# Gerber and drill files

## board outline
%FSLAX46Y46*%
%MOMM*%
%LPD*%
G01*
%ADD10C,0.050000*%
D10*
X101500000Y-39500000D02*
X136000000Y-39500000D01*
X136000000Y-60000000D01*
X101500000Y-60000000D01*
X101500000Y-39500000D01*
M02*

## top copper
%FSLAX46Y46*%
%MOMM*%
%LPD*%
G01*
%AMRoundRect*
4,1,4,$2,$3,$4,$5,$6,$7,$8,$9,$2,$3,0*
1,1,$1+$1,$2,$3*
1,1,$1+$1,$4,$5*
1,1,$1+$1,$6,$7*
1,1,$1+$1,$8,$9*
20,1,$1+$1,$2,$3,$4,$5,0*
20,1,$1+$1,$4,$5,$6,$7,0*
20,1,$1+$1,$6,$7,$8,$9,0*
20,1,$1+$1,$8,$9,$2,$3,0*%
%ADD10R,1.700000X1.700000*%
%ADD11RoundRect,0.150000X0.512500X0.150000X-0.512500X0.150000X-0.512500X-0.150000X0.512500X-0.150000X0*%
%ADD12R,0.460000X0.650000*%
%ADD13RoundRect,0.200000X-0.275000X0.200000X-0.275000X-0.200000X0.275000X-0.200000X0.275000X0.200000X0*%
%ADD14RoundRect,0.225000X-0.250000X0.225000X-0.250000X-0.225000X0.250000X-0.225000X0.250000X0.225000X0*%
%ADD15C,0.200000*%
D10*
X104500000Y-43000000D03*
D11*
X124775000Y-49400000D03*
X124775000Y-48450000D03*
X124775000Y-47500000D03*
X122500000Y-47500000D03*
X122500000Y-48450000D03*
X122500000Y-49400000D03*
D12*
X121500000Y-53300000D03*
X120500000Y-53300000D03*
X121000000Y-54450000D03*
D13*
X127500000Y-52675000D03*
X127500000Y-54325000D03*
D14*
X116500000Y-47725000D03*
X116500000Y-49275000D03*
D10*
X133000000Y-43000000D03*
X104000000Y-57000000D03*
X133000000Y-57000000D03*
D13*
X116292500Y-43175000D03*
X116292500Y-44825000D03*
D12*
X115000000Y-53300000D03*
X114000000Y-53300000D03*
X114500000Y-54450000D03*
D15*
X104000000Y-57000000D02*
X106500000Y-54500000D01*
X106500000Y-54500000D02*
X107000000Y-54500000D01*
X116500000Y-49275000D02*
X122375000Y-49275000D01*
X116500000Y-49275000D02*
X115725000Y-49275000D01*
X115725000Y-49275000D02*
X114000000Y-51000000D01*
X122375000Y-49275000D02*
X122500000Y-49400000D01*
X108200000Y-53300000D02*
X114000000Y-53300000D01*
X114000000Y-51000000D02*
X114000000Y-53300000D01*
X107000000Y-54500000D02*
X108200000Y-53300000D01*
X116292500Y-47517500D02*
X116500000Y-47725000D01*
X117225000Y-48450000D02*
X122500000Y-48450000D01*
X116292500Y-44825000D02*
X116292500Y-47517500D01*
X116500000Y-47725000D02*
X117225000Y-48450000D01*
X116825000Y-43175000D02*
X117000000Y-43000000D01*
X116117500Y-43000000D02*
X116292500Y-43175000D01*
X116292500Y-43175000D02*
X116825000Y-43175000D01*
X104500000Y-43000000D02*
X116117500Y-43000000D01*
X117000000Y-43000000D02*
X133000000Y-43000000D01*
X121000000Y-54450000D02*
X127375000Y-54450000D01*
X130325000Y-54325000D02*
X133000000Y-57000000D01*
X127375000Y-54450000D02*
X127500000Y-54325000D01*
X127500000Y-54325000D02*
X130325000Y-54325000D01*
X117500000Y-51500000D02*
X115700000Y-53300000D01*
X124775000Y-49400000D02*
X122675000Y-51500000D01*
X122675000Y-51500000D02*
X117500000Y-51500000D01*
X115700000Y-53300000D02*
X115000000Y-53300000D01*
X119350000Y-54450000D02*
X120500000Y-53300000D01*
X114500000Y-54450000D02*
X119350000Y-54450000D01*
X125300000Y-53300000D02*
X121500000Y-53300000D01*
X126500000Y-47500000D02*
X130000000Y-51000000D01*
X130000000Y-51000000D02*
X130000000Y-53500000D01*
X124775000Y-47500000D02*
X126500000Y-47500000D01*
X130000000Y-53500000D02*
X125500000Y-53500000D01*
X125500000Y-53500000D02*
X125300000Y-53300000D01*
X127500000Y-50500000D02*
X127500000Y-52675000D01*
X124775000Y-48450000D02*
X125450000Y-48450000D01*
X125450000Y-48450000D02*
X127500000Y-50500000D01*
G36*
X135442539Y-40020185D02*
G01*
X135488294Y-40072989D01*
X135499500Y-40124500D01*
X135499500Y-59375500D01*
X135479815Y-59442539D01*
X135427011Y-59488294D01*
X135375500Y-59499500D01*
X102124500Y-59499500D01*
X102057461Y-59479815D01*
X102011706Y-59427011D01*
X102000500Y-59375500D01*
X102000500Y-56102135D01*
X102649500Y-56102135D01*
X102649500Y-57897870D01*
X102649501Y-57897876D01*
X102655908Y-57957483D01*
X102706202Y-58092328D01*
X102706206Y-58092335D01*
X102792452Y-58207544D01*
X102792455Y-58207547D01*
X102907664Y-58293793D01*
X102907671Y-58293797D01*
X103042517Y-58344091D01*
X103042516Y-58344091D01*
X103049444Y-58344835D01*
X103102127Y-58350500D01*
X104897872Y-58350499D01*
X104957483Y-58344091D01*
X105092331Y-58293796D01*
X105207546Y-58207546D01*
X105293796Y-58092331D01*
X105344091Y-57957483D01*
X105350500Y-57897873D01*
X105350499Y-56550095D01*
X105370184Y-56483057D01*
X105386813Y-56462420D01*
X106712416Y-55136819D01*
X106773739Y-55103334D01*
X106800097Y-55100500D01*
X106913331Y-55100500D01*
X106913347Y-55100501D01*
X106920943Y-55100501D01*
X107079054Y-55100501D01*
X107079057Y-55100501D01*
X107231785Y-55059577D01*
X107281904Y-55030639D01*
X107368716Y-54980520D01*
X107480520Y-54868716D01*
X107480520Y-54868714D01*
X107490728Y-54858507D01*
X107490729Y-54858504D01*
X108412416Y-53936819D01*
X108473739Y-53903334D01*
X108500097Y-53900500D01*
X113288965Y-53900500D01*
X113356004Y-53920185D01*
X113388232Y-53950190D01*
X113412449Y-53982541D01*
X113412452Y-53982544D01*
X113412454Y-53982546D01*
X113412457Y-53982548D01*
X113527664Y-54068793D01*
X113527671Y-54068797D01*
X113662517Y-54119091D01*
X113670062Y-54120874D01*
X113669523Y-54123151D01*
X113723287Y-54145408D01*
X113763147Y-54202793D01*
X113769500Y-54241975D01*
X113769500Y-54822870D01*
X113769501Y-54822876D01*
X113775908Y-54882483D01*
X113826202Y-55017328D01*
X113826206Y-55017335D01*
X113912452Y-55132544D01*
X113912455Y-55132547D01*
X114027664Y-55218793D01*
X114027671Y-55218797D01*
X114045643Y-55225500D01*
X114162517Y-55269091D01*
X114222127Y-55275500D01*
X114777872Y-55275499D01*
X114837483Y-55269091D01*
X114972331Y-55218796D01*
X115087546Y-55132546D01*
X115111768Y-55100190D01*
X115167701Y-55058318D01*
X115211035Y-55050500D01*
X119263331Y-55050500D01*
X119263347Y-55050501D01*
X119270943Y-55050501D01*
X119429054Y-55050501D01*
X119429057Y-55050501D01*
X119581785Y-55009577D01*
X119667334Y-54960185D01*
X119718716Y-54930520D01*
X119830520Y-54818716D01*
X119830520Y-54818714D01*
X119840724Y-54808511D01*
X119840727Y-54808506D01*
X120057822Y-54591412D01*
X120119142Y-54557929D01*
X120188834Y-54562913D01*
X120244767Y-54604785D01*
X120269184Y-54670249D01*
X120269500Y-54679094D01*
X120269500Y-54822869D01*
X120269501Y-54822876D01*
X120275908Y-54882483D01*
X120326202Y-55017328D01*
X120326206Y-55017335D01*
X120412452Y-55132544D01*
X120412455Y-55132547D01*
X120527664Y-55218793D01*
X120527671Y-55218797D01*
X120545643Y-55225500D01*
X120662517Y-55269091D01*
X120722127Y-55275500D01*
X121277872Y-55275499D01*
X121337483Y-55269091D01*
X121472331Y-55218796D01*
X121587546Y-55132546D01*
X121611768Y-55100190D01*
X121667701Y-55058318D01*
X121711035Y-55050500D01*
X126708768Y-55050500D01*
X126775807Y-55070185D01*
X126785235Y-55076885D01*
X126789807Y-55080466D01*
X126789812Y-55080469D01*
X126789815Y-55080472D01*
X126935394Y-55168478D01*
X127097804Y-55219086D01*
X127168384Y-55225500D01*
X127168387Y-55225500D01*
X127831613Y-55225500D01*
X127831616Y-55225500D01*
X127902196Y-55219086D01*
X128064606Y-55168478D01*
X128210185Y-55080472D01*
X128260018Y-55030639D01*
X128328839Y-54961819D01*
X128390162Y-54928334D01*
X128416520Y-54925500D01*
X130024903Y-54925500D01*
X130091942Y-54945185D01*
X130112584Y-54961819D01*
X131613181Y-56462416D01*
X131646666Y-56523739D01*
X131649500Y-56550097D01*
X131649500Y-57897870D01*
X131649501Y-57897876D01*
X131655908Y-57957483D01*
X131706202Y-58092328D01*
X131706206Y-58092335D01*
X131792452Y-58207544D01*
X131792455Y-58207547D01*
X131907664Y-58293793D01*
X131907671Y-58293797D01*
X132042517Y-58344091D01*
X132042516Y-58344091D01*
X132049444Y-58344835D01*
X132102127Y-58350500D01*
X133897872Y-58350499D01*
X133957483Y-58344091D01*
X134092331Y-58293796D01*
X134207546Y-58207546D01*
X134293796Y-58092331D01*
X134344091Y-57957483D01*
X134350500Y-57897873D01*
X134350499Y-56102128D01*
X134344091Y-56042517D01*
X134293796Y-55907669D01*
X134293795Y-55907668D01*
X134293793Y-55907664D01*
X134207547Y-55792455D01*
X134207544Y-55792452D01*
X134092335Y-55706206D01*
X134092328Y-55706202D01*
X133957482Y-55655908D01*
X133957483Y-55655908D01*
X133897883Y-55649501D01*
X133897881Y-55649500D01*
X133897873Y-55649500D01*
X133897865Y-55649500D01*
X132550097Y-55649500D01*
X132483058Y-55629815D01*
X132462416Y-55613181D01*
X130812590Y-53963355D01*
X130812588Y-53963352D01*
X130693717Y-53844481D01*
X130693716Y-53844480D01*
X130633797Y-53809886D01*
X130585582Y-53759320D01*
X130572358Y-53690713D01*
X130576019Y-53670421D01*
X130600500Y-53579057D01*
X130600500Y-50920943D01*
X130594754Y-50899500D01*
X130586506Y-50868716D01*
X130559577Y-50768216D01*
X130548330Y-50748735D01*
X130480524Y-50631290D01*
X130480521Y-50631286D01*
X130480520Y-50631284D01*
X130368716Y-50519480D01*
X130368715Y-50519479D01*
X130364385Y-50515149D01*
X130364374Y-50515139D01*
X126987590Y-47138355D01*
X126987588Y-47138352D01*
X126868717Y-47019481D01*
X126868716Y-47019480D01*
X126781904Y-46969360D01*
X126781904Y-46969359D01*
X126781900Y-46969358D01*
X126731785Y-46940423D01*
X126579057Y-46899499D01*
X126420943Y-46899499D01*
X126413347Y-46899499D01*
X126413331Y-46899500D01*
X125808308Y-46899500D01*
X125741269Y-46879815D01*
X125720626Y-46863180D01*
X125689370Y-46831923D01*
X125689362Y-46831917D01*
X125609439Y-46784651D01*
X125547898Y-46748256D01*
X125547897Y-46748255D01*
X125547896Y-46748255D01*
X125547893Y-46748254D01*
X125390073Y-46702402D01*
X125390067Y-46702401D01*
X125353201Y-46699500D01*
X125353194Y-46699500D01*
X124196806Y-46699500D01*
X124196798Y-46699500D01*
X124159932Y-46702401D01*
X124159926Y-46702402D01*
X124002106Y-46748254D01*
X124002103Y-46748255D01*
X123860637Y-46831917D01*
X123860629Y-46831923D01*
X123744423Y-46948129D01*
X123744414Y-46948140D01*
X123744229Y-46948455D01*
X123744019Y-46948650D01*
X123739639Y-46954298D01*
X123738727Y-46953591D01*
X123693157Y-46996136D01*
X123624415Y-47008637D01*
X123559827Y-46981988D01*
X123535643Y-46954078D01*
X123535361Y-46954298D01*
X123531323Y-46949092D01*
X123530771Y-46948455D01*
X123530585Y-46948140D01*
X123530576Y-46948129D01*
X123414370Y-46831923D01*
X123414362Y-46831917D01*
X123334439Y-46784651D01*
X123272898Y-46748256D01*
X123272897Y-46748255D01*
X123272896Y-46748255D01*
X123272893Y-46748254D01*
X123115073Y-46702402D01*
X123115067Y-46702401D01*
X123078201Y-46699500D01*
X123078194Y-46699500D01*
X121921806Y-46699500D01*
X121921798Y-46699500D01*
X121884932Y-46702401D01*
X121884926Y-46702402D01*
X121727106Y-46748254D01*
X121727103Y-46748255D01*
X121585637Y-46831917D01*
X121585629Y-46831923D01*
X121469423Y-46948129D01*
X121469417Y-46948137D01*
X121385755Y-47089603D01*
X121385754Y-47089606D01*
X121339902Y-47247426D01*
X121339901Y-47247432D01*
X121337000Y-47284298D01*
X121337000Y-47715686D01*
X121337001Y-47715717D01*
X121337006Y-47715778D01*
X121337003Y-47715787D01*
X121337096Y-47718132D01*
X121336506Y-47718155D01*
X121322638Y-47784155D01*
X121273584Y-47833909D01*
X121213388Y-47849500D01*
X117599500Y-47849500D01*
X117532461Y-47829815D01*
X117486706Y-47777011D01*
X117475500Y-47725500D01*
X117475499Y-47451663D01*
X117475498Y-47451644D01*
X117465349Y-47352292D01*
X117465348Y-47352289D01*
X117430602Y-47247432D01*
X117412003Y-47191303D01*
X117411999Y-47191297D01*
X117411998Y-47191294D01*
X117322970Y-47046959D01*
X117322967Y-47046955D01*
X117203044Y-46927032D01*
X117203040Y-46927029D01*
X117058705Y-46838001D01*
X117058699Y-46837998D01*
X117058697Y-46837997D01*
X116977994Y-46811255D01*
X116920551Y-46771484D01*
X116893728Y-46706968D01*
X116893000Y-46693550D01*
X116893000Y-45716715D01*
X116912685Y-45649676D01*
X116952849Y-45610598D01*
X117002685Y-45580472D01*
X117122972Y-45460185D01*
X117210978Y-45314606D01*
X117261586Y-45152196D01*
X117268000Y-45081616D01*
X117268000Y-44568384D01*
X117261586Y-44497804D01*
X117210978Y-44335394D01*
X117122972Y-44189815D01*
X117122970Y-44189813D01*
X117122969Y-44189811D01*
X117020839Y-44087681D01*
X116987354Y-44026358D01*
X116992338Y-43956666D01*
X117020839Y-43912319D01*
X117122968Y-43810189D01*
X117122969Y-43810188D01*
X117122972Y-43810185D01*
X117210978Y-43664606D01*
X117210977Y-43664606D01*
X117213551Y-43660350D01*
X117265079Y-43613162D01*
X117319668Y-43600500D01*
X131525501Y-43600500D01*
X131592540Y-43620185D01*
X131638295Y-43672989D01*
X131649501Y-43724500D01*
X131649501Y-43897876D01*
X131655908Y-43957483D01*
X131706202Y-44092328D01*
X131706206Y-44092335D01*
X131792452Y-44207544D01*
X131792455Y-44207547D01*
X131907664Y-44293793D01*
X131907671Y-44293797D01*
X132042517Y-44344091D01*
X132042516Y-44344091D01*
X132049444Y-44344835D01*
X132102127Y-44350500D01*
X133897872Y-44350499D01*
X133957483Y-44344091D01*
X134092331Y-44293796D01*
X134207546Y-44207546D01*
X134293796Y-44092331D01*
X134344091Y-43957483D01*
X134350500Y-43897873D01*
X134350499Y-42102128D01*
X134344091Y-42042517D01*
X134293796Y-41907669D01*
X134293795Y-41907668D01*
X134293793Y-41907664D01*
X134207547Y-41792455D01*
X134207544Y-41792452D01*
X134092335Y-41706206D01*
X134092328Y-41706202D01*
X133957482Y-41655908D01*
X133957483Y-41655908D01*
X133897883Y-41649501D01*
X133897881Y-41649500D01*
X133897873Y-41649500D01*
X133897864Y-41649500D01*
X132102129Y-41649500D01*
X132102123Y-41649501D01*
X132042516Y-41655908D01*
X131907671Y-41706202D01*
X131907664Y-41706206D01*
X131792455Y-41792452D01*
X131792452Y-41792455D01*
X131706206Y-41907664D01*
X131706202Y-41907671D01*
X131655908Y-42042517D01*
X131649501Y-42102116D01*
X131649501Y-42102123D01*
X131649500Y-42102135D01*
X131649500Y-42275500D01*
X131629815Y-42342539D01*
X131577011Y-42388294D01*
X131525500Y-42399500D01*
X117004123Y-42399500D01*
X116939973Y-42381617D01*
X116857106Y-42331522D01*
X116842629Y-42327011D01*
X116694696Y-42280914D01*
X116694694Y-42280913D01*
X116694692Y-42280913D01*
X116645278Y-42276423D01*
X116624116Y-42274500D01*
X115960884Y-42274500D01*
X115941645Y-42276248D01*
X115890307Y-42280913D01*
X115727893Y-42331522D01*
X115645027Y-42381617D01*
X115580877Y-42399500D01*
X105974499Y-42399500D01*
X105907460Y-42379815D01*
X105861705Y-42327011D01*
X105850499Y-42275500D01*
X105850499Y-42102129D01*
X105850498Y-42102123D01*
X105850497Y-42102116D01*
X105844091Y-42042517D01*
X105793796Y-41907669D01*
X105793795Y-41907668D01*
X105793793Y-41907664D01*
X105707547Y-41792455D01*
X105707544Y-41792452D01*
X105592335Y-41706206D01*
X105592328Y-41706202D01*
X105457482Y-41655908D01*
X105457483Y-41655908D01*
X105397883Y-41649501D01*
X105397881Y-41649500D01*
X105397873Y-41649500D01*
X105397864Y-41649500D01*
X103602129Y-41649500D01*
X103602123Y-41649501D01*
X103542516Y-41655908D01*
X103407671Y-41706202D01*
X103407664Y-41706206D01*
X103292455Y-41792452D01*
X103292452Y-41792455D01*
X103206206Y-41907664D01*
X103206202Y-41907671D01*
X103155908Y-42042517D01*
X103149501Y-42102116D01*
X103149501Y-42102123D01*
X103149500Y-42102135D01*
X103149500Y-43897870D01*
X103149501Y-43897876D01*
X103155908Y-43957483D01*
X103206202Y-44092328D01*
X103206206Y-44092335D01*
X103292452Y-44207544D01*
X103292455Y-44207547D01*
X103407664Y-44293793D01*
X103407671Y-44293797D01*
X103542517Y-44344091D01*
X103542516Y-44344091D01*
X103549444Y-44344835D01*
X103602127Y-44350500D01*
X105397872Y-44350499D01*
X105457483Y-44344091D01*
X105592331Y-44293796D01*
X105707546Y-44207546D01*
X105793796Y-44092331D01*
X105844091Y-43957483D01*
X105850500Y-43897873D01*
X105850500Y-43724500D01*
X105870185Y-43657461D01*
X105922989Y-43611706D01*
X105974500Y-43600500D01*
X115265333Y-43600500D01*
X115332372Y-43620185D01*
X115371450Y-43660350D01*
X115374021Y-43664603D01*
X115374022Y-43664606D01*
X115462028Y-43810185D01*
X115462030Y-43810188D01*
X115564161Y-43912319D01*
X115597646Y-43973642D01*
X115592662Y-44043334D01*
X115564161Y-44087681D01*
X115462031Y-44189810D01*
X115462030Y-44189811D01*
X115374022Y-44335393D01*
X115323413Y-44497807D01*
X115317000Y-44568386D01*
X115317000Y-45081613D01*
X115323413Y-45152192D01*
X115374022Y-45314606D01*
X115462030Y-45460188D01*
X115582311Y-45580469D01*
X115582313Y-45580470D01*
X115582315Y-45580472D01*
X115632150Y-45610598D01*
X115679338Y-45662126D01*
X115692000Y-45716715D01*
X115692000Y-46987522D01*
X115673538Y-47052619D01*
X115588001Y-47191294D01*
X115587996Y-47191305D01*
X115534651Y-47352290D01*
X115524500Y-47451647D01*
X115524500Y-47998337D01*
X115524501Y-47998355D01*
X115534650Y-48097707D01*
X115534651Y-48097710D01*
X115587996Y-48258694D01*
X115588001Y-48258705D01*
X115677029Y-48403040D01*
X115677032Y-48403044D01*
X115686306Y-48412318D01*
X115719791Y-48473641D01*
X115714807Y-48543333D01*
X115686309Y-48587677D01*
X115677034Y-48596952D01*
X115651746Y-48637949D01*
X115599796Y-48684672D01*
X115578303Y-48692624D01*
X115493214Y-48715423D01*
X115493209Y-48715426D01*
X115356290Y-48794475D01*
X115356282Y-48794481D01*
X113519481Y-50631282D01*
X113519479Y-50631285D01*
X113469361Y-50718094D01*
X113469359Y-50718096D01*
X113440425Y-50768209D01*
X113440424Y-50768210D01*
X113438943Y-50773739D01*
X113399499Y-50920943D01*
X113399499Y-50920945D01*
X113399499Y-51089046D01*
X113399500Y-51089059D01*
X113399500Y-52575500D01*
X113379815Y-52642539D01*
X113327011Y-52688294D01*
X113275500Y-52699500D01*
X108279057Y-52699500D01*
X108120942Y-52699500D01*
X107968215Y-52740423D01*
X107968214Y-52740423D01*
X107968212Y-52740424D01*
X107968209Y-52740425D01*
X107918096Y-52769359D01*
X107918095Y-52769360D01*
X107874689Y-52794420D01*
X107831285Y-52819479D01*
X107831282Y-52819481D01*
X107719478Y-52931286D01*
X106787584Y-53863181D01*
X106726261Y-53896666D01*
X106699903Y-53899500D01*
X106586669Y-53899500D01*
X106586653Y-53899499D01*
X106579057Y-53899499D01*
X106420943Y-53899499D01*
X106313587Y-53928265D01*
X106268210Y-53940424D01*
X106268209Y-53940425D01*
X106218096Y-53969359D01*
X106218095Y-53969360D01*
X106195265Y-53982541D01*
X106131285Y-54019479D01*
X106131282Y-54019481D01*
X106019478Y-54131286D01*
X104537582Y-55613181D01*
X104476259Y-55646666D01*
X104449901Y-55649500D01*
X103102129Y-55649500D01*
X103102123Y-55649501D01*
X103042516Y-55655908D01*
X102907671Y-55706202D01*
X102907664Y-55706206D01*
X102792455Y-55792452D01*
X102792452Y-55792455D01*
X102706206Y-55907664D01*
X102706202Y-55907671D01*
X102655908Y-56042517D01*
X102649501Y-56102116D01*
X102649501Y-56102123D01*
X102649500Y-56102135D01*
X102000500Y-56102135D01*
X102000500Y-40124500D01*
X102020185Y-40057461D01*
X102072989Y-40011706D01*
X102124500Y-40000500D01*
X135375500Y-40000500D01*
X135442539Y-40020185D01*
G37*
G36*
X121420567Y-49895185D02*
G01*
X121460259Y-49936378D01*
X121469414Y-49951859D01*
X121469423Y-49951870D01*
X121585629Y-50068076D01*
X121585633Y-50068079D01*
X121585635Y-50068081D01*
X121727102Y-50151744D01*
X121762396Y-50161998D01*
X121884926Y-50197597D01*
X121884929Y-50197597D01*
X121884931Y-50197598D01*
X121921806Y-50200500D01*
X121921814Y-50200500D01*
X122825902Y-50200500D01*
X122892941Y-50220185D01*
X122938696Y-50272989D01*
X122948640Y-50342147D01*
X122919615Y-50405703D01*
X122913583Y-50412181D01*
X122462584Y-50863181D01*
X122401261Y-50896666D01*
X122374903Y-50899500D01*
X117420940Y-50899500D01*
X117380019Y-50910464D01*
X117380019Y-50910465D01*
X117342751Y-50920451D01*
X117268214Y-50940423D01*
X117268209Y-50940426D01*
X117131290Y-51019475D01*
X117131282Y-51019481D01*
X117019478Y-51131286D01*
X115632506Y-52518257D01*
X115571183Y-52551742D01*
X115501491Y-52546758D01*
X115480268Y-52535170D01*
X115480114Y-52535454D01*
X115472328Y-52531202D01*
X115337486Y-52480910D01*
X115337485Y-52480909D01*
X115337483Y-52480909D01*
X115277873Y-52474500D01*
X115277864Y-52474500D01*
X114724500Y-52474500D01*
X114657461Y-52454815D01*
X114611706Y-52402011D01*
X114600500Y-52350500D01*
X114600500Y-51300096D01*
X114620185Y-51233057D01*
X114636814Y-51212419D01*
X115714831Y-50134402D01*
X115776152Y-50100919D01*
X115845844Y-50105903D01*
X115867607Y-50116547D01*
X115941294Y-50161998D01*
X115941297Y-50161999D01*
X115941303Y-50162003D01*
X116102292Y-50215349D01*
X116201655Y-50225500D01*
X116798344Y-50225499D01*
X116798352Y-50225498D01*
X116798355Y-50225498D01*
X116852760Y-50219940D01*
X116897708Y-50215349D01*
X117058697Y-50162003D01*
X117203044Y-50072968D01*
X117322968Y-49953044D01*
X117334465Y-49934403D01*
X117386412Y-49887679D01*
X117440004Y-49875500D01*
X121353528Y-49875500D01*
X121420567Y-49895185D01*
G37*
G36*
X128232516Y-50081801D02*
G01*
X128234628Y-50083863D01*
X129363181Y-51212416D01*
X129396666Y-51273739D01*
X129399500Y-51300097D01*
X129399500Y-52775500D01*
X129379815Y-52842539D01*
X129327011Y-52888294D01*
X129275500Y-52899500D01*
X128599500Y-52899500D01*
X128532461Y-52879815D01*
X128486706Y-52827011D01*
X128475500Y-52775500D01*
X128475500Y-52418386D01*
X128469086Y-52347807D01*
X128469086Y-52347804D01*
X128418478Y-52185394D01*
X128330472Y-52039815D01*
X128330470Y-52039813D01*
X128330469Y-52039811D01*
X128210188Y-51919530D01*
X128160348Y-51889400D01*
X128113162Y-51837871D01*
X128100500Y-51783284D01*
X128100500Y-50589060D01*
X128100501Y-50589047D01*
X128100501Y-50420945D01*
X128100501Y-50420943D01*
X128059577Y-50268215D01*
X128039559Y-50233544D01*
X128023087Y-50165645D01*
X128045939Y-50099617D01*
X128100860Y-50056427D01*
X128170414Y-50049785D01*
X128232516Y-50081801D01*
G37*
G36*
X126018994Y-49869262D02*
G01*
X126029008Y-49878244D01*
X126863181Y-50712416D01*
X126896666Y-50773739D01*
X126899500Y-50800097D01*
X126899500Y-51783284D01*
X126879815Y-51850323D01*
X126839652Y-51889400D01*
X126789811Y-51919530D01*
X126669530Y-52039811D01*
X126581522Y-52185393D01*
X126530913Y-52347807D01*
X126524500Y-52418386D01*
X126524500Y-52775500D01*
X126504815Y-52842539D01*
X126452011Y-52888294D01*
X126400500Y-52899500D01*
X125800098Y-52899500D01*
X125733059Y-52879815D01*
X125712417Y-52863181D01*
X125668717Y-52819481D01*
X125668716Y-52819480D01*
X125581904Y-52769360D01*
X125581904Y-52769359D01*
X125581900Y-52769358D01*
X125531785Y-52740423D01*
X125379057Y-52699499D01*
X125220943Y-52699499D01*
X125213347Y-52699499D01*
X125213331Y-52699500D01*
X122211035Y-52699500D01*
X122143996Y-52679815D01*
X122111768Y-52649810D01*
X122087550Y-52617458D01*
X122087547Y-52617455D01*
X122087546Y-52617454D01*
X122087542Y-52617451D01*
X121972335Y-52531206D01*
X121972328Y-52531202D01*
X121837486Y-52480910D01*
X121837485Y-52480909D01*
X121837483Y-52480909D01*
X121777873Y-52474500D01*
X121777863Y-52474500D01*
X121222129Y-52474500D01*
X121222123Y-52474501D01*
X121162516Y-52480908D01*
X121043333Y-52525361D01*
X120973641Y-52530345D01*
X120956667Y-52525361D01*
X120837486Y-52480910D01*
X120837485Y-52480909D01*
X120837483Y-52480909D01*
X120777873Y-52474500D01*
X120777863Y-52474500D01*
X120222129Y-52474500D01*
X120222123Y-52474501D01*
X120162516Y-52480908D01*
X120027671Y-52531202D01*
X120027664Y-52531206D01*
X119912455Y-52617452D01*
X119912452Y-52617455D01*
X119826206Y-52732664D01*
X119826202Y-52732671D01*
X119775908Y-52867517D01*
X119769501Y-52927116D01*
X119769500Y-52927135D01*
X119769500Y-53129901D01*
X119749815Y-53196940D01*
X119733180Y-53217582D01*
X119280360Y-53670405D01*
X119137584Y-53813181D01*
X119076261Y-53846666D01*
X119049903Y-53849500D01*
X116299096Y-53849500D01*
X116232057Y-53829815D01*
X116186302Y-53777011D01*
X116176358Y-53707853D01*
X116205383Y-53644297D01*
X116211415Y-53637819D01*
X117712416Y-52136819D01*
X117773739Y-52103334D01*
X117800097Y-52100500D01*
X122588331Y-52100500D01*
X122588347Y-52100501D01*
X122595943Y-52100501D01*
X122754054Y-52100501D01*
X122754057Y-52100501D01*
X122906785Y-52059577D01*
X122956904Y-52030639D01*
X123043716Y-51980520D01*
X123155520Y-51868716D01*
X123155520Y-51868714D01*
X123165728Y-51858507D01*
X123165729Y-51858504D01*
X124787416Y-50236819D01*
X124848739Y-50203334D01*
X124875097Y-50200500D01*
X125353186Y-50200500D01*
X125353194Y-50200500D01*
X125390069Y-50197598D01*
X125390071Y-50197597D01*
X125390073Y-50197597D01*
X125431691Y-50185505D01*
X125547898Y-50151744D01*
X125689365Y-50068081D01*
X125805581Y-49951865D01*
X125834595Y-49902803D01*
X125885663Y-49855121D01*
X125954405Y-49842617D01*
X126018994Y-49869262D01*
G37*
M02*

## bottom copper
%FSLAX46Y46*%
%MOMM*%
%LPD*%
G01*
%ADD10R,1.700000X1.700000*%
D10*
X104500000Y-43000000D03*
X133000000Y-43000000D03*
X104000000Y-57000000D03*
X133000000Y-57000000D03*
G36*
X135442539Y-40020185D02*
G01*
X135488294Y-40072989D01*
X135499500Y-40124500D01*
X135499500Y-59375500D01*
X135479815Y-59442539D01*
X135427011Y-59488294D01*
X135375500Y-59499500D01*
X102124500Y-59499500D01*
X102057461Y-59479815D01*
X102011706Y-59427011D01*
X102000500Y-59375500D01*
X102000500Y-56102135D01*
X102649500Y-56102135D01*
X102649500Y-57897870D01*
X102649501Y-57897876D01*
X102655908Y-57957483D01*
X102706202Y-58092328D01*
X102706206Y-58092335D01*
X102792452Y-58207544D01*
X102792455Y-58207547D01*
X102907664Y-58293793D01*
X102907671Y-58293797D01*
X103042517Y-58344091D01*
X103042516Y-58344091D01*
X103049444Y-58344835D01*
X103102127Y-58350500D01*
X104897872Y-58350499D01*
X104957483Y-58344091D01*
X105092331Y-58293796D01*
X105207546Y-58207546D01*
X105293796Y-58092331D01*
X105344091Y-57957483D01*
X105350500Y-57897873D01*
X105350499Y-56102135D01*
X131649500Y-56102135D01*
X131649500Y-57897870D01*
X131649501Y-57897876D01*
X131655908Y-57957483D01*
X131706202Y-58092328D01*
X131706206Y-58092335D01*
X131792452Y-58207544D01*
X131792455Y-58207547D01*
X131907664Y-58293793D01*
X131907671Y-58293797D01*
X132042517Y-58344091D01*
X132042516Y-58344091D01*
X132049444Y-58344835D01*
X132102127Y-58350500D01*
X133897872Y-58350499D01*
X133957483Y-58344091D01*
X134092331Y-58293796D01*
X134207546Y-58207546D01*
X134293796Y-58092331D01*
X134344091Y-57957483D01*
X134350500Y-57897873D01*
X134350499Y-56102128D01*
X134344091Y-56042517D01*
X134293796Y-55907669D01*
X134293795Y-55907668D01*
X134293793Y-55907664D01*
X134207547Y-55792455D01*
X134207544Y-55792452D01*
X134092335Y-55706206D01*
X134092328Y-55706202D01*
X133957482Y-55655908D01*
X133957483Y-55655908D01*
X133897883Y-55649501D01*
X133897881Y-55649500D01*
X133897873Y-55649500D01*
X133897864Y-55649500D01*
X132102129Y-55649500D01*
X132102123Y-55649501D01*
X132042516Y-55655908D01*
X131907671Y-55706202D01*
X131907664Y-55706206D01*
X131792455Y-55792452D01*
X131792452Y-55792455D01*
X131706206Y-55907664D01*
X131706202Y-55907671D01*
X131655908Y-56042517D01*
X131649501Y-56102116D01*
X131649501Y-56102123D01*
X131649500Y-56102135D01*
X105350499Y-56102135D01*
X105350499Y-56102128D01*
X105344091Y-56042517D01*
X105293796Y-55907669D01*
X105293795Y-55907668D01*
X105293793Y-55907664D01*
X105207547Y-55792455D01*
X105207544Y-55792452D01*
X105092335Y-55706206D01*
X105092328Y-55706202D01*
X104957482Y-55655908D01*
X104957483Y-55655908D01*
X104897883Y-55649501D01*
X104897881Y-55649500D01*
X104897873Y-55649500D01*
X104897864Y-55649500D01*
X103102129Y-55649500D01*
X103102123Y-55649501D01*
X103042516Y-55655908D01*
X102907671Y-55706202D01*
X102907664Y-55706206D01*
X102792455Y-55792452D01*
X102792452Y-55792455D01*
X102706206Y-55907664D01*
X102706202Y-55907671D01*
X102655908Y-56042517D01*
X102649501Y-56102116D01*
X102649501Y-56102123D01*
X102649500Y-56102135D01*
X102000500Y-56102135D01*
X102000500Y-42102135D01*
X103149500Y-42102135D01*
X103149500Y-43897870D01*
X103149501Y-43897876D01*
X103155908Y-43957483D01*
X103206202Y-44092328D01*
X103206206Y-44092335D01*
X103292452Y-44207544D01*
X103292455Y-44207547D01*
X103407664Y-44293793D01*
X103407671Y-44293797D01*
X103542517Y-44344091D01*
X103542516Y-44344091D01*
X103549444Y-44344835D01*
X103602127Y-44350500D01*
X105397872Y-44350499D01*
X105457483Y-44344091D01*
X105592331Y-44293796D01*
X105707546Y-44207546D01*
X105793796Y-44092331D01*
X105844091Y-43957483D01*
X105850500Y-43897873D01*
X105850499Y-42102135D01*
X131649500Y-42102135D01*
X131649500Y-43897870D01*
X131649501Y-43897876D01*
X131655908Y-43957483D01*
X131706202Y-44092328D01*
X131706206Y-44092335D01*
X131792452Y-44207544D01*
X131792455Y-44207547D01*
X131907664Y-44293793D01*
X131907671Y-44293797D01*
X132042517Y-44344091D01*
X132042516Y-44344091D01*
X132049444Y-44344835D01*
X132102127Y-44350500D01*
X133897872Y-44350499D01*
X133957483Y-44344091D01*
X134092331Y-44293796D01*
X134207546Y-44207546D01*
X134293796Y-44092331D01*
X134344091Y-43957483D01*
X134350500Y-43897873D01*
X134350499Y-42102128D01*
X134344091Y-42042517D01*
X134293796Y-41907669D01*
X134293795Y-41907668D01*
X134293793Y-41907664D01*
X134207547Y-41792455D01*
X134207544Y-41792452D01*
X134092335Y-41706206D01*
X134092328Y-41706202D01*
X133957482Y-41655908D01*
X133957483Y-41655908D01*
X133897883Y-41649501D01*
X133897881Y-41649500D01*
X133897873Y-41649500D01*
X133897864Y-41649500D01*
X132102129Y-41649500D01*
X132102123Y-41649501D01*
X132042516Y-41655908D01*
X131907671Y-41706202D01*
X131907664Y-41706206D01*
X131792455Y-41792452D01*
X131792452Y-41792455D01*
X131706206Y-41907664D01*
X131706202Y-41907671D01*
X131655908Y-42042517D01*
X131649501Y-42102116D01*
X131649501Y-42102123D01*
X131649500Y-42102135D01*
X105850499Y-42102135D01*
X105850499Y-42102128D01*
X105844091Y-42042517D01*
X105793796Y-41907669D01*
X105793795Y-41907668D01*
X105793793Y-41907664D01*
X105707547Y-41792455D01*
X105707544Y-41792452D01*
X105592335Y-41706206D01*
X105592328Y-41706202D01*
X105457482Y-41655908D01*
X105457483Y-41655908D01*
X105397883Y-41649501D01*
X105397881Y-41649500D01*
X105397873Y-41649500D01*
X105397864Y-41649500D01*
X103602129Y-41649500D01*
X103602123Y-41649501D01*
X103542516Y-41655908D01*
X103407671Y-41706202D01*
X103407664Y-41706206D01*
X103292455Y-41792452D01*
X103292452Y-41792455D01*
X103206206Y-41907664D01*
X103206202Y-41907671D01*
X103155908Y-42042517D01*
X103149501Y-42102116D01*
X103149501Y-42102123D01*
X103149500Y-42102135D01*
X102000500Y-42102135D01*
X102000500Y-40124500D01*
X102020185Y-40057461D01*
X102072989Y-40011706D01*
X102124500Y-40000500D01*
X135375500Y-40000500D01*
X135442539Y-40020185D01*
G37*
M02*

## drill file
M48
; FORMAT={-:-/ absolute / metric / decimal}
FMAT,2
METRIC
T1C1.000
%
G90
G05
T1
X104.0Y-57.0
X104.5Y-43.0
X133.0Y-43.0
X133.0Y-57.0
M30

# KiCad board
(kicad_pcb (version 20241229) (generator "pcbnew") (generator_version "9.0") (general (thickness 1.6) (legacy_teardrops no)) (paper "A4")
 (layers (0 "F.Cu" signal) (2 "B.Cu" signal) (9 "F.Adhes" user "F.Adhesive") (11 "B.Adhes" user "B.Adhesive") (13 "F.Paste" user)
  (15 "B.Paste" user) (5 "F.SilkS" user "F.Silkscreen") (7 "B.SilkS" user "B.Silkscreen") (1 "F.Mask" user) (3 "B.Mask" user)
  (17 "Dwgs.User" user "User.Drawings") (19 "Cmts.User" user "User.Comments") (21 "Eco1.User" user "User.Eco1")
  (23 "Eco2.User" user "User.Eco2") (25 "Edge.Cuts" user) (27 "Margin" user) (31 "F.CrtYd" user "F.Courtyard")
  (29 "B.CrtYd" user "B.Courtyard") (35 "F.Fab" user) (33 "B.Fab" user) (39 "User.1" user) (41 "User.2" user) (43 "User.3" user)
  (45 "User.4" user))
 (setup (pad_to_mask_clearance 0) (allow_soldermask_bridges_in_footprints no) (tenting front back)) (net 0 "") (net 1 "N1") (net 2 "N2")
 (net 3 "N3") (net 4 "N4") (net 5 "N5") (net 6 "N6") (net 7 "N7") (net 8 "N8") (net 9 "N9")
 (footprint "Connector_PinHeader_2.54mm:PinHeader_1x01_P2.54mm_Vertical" (layer "F.Cu") (at 104.5 43)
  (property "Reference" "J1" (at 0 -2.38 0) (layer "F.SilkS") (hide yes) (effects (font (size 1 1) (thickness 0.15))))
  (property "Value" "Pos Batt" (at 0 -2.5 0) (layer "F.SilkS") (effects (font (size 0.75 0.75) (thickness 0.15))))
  (pad "1" thru_hole rect (at 0 0) (size 1.7 1.7) (drill 1) (layers "*.Cu" "*.Mask") (remove_unused_layers no) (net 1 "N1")))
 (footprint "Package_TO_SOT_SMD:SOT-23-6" (layer "F.Cu") (at 123.6375 48.45 180)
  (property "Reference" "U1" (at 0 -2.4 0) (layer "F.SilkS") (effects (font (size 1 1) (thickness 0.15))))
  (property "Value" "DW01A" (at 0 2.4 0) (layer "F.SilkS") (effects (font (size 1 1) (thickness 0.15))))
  (pad "1" smd roundrect (at -1.1375 -0.95 180) (size 1.325 0.6) (layers "F.Cu" "F.Mask" "F.Paste") (roundrect_rratio 0.25) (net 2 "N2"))
  (pad "2" smd roundrect (at -1.1375 0 180) (size 1.325 0.6) (layers "F.Cu" "F.Mask" "F.Paste") (roundrect_rratio 0.25) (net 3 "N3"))
  (pad "3" smd roundrect (at -1.1375 0.95 180) (size 1.325 0.6) (layers "F.Cu" "F.Mask" "F.Paste") (roundrect_rratio 0.25) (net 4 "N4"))
  (pad "4" smd roundrect (at 1.1375 0.95 180) (size 1.325 0.6) (layers "F.Cu" "F.Mask" "F.Paste") (roundrect_rratio 0.25) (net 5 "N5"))
  (pad "5" smd roundrect (at 1.1375 0 180) (size 1.325 0.6) (layers "F.Cu" "F.Mask" "F.Paste") (roundrect_rratio 0.25) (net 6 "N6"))
  (pad "6" smd roundrect (at 1.1375 -0.95 180) (size 1.325 0.6) (layers "F.Cu" "F.Mask" "F.Paste") (roundrect_rratio 0.25) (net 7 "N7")))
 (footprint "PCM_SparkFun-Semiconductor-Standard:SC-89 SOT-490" (layer "F.Cu") (at 121 54.4 180)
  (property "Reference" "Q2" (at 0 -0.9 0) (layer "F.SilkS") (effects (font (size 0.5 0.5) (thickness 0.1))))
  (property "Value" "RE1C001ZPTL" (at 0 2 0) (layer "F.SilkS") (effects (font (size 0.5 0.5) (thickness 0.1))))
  (pad "1" smd rect (at -0.5 1.1 180) (size 0.46 0.65) (layers "F.Cu" "F.Mask" "F.Paste") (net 4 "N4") (thermal_bridge_angle 0))
  (pad "2" smd rect (at 0.5 1.1 180) (size 0.46 0.65) (layers "F.Cu" "F.Mask" "F.Paste") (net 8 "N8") (thermal_bridge_angle 0))
  (pad "3" smd rect (at 0 -0.05 180) (size 0.46 0.65) (layers "F.Cu" "F.Mask" "F.Paste") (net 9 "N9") (thermal_bridge_angle 0)))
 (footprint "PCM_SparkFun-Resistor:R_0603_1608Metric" (layer "F.Cu") (at 127.5 53.5 -90)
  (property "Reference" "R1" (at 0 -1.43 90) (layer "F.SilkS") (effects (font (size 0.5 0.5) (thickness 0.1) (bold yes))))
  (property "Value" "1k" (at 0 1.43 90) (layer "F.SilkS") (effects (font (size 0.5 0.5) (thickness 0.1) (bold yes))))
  (pad "1" smd roundrect (at -0.825 0 270) (size 0.8 0.95) (layers "F.Cu" "F.Mask" "F.Paste") (roundrect_rratio 0.25) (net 3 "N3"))
  (pad "2" smd roundrect (at 0.825 0 270) (size 0.8 0.95) (layers "F.Cu" "F.Mask" "F.Paste") (roundrect_rratio 0.25) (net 9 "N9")))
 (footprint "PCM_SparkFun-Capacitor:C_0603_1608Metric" (layer "F.Cu") (at 116.5 48.5 -90)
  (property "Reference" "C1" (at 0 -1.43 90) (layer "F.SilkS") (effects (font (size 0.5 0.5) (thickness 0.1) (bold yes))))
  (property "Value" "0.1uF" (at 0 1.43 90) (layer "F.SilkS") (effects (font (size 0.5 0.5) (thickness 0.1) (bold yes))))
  (pad "1" smd roundrect (at -0.775 0 270) (size 0.9 0.95) (layers "F.Cu" "F.Mask" "F.Paste") (roundrect_rratio 0.25) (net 6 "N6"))
  (pad "2" smd roundrect (at 0.775 0 270) (size 0.9 0.95) (layers "F.Cu" "F.Mask" "F.Paste") (roundrect_rratio 0.25) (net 7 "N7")))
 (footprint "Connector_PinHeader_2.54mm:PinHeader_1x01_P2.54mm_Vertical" (layer "F.Cu") (at 133 43)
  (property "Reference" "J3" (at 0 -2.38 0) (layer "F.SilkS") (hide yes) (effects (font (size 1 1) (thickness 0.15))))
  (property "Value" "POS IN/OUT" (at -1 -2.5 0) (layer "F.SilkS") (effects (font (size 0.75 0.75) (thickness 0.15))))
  (pad "1" thru_hole rect (at 0 0) (size 1.7 1.7) (drill 1) (layers "*.Cu" "*.Mask") (remove_unused_layers no) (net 1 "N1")))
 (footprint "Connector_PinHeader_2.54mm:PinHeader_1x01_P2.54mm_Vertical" (layer "F.Cu") (at 104 57)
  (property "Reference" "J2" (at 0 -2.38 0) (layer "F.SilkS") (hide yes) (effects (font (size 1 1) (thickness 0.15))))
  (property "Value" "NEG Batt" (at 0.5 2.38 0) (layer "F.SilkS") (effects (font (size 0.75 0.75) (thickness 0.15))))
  (pad "1" thru_hole rect (at 0 0) (size 1.7 1.7) (drill 1) (layers "*.Cu" "*.Mask") (remove_unused_layers no) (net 7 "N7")))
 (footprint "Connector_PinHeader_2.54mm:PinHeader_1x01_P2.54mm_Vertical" (layer "F.Cu") (at 133 57)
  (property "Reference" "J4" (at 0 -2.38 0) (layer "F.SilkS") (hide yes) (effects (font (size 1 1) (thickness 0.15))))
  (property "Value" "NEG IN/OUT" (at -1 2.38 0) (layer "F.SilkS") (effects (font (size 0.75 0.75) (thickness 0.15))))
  (pad "1" thru_hole rect (at 0 0) (size 1.7 1.7) (drill 1) (layers "*.Cu" "*.Mask") (remove_unused_layers no) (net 9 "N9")))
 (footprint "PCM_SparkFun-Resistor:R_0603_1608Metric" (layer "F.Cu") (at 116.2925 44 -90)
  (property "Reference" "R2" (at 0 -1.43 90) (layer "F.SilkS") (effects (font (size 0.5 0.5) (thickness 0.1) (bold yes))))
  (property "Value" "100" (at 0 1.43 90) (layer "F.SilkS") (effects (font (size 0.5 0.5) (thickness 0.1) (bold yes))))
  (pad "1" smd roundrect (at -0.825 0 270) (size 0.8 0.95) (layers "F.Cu" "F.Mask" "F.Paste") (roundrect_rratio 0.25) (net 1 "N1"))
  (pad "2" smd roundrect (at 0.825 0 270) (size 0.8 0.95) (layers "F.Cu" "F.Mask" "F.Paste") (roundrect_rratio 0.25) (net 6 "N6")))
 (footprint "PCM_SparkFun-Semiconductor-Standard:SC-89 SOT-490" (layer "F.Cu") (at 114.5 54.4 180)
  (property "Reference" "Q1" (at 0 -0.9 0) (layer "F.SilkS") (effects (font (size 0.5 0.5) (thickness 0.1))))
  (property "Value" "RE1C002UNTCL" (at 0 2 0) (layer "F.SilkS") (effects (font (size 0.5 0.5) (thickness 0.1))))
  (pad "1" smd rect (at -0.5 1.1 180) (size 0.46 0.65) (layers "F.Cu" "F.Mask" "F.Paste") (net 2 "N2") (thermal_bridge_angle 0))
  (pad "2" smd rect (at 0.5 1.1 180) (size 0.46 0.65) (layers "F.Cu" "F.Mask" "F.Paste") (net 7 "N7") (thermal_bridge_angle 0))
  (pad "3" smd rect (at 0 -0.05 180) (size 0.46 0.65) (layers "F.Cu" "F.Mask" "F.Paste") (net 8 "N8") (thermal_bridge_angle 0)))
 (gr_rect (start 101.5 39.5) (end 136 60) (stroke (width 0.05) (type default)) (fill no) (layer "Edge.Cuts"))
 (segment (start 104 57) (end 106.5 54.5) (width 0.2) (layer "F.Cu") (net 7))
 (segment (start 106.5 54.5) (end 107 54.5) (width 0.2) (layer "F.Cu") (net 7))
 (segment (start 116.5 49.275) (end 122.375 49.275) (width 0.2) (layer "F.Cu") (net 7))
 (segment (start 116.5 49.275) (end 115.725 49.275) (width 0.2) (layer "F.Cu") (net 7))
 (segment (start 115.725 49.275) (end 114 51) (width 0.2) (layer "F.Cu") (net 7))
 (segment (start 122.375 49.275) (end 122.5 49.4) (width 0.2) (layer "F.Cu") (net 7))
 (segment (start 108.2 53.3) (end 114 53.3) (width 0.2) (layer "F.Cu") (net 7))
 (segment (start 114 51) (end 114 53.3) (width 0.2) (layer "F.Cu") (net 7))
 (segment (start 107 54.5) (end 108.2 53.3) (width 0.2) (layer "F.Cu") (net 7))
 (segment (start 116.2925 47.5175) (end 116.5 47.725) (width 0.2) (layer "F.Cu") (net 6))
 (segment (start 117.225 48.45) (end 122.5 48.45) (width 0.2) (layer "F.Cu") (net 6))
 (segment (start 116.2925 44.825) (end 116.2925 47.5175) (width 0.2) (layer "F.Cu") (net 6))
 (segment (start 116.5 47.725) (end 117.225 48.45) (width 0.2) (layer "F.Cu") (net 6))
 (segment (start 116.825 43.175) (end 117 43) (width 0.2) (layer "F.Cu") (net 1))
 (segment (start 116.1175 43) (end 116.2925 43.175) (width 0.2) (layer "F.Cu") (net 1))
 (segment (start 116.2925 43.175) (end 116.825 43.175) (width 0.2) (layer "F.Cu") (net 1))
 (segment (start 104.5 43) (end 116.1175 43) (width 0.2) (layer "F.Cu") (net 1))
 (segment (start 117 43) (end 133 43) (width 0.2) (layer "F.Cu") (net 1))
 (segment (start 121 54.45) (end 127.375 54.45) (width 0.2) (layer "F.Cu") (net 9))
 (segment (start 130.325 54.325) (end 133 57) (width 0.2) (layer "F.Cu") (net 9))
 (segment (start 127.375 54.45) (end 127.5 54.325) (width 0.2) (layer "F.Cu") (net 9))
 (segment (start 127.5 54.325) (end 130.325 54.325) (width 0.2) (layer "F.Cu") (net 9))
 (segment (start 117.5 51.5) (end 115.7 53.3) (width 0.2) (layer "F.Cu") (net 2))
 (segment (start 124.775 49.4) (end 122.675 51.5) (width 0.2) (layer "F.Cu") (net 2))
 (segment (start 122.675 51.5) (end 117.5 51.5) (width 0.2) (layer "F.Cu") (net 2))
 (segment (start 115.7 53.3) (end 115 53.3) (width 0.2) (layer "F.Cu") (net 2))
 (segment (start 119.35 54.45) (end 120.5 53.3) (width 0.2) (layer "F.Cu") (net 8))
 (segment (start 114.5 54.45) (end 119.35 54.45) (width 0.2) (layer "F.Cu") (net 8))
 (segment (start 125.3 53.3) (end 121.5 53.3) (width 0.2) (layer "F.Cu") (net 4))
 (segment (start 126.5 47.5) (end 130 51) (width 0.2) (layer "F.Cu") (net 4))
 (segment (start 130 51) (end 130 53.5) (width 0.2) (layer "F.Cu") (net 4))
 (segment (start 124.775 47.5) (end 126.5 47.5) (width 0.2) (layer "F.Cu") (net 4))
 (segment (start 130 53.5) (end 125.5 53.5) (width 0.2) (layer "F.Cu") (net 4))
 (segment (start 125.5 53.5) (end 125.3 53.3) (width 0.2) (layer "F.Cu") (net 4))
 (segment (start 127.5 50.5) (end 127.5 52.675) (width 0.2) (layer "F.Cu") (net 3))
 (segment (start 124.775 48.45) (end 125.45 48.45) (width 0.2) (layer "F.Cu") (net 3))
 (segment (start 125.45 48.45) (end 127.5 50.5) (width 0.2) (layer "F.Cu") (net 3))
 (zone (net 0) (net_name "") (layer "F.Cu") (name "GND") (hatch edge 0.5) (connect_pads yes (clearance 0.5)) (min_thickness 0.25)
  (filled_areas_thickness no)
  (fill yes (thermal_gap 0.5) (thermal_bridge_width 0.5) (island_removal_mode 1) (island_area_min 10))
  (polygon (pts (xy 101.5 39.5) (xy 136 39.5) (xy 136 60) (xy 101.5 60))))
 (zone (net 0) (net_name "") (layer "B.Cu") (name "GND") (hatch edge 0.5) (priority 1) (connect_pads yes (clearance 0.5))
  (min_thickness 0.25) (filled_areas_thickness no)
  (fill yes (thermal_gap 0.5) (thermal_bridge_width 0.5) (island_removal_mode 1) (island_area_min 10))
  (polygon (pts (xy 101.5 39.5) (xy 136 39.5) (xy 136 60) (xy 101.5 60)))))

